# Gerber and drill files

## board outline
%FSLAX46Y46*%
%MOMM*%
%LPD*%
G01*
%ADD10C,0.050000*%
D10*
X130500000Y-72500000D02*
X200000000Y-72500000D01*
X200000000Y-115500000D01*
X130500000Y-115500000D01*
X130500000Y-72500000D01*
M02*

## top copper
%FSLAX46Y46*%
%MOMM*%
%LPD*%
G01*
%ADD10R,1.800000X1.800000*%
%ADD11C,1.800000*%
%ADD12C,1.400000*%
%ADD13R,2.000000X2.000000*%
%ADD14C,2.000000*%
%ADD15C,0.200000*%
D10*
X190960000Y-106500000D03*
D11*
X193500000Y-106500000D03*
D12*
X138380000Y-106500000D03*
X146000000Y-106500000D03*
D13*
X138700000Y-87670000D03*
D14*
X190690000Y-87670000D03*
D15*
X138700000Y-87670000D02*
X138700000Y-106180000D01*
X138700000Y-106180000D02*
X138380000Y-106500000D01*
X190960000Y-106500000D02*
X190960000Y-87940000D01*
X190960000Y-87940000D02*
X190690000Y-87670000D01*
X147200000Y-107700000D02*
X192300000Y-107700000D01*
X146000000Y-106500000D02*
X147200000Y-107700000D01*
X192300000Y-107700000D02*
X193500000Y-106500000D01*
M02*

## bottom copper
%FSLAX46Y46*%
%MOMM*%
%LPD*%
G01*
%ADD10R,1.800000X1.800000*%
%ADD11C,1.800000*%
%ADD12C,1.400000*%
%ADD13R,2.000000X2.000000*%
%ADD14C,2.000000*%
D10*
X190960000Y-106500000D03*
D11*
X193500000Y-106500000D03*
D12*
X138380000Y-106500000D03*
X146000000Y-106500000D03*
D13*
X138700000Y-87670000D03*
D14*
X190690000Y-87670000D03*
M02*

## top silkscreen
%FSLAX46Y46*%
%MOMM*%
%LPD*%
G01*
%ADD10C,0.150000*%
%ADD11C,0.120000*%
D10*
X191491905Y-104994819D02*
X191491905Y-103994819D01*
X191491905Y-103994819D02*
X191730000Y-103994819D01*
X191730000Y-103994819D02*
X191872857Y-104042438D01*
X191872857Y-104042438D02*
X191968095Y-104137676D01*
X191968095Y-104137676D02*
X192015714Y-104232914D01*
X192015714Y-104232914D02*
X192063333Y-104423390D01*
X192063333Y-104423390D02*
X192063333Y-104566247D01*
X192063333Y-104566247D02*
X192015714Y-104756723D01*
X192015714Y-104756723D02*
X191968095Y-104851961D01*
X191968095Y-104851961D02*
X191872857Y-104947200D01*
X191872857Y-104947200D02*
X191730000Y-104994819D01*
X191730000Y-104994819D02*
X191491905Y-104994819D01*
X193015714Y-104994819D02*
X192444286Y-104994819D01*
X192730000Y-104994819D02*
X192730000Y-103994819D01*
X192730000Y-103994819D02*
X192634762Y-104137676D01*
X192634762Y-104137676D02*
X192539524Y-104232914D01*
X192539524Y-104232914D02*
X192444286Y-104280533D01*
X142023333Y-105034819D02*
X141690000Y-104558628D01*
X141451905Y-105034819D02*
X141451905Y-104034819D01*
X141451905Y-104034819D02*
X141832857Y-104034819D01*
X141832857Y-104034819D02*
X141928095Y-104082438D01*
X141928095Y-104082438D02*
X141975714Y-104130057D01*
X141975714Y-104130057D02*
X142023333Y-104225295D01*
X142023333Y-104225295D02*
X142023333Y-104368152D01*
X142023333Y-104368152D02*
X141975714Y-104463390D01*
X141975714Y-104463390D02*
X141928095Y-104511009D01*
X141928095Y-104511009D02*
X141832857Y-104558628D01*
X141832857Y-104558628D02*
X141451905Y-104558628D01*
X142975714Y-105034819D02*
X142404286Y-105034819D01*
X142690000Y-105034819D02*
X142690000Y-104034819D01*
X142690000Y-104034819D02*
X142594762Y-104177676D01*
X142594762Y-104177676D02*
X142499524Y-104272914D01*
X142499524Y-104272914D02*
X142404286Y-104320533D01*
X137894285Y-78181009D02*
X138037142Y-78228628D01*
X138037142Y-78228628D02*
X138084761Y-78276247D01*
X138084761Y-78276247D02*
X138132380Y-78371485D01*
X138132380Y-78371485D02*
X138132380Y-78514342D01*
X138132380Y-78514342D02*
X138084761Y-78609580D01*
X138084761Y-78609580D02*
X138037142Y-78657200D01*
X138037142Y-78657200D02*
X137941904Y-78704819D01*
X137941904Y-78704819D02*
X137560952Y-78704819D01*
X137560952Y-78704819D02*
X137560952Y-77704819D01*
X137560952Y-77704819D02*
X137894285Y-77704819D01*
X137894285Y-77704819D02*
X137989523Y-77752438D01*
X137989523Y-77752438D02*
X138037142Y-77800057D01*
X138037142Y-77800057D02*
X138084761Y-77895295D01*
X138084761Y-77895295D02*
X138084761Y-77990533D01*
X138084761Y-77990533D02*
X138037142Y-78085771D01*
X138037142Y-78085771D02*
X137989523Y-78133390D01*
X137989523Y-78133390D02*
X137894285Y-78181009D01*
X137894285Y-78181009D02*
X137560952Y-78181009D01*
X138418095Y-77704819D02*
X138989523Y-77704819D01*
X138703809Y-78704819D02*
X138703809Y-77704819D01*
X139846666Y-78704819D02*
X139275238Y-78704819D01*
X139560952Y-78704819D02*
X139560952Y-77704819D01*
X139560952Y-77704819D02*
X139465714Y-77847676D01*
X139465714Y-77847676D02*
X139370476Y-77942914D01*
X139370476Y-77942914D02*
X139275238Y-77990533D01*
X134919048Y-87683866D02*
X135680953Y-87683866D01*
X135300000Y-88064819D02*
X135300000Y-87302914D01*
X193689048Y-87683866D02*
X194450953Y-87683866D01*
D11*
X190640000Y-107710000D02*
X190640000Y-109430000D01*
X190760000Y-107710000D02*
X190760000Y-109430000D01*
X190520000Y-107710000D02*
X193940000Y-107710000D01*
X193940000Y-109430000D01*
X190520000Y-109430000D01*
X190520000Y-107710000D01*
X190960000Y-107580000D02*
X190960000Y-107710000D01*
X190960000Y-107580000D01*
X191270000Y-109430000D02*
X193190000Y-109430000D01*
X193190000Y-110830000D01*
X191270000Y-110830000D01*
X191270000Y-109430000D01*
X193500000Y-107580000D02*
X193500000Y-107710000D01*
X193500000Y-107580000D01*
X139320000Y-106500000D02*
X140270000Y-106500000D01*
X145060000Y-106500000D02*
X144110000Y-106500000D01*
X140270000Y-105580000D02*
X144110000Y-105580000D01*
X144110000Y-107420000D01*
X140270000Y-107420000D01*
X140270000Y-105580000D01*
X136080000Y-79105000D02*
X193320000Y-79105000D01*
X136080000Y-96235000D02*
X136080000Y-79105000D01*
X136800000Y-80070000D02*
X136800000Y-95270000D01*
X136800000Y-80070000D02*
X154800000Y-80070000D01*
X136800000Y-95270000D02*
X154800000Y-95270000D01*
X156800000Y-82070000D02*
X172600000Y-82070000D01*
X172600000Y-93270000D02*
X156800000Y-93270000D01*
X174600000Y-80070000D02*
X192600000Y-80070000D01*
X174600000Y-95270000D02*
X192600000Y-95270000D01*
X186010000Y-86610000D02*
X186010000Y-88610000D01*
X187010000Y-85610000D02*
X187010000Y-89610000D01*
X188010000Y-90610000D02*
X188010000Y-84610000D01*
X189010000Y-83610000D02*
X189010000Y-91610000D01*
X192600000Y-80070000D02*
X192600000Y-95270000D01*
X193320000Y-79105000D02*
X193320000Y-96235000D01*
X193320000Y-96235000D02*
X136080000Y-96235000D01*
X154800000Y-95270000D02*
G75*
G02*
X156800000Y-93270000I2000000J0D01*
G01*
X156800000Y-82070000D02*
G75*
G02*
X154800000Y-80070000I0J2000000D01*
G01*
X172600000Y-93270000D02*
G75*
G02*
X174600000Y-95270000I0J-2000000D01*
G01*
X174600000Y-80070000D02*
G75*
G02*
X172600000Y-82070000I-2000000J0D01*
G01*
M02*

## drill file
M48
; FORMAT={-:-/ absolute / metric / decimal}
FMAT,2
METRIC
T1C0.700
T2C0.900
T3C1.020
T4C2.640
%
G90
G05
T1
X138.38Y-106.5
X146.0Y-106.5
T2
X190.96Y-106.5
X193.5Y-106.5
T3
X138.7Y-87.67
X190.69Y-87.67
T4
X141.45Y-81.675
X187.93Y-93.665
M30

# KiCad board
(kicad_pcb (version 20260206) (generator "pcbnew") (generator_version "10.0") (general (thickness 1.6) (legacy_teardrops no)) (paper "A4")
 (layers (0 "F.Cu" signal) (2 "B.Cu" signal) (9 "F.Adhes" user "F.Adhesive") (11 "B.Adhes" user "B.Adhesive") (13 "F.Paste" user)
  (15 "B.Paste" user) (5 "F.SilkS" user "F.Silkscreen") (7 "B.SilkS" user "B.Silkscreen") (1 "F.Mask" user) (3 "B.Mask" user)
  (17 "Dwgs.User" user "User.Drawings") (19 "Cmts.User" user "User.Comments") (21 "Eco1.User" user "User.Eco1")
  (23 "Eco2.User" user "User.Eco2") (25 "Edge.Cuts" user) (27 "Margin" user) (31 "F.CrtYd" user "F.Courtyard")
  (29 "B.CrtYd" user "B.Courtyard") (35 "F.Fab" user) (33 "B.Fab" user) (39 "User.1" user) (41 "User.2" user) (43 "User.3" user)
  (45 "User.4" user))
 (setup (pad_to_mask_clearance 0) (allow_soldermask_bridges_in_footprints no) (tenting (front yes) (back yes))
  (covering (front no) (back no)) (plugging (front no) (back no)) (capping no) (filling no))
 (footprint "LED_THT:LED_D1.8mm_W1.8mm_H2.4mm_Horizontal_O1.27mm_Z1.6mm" (layer "F.Cu") (at 190.96 106.5)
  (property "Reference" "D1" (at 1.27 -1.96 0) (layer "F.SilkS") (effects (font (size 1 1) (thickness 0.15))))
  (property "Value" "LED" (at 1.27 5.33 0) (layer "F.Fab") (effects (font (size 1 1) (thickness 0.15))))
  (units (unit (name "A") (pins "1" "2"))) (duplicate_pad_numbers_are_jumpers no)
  (fp_line (start -0.32 1.21) (end -0.32 2.93) (stroke (width 0.12) (type solid)) (layer "F.SilkS"))
  (fp_line (start -0.2 1.21) (end -0.2 2.93) (stroke (width 0.12) (type solid)) (layer "F.SilkS"))
  (fp_rect (start -0.44 1.21) (end 2.98 2.93) (stroke (width 0.12) (type solid)) (fill no) (layer "F.SilkS"))
  (fp_rect (start 0 1.08) (end 0 1.21) (stroke (width 0.12) (type solid)) (fill no) (layer "F.SilkS"))
  (fp_rect (start 0.31 2.93) (end 2.23 4.33) (stroke (width 0.12) (type solid)) (fill no) (layer "F.SilkS"))
  (fp_rect (start 2.54 1.08) (end 2.54 1.21) (stroke (width 0.12) (type solid)) (fill no) (layer "F.SilkS"))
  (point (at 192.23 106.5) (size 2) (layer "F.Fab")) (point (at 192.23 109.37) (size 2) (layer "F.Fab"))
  (pad "1" thru_hole rect (at 0 0) (size 1.8 1.8) (drill 0.9) (layers "*.Cu" "*.Mask") (remove_unused_layers no) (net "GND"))
  (pad "2" thru_hole circle (at 2.54 0) (size 1.8 1.8) (drill 0.9) (layers "*.Cu" "*.Mask") (remove_unused_layers no) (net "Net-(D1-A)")))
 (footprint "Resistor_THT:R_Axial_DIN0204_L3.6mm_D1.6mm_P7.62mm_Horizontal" (layer "F.Cu") (at 138.38 106.5)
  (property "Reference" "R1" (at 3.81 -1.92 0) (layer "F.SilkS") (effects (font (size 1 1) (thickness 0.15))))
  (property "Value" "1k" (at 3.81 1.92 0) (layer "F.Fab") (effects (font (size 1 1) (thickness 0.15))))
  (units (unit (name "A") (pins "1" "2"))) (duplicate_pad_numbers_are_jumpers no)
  (fp_line (start 0.94 0) (end 1.89 0) (stroke (width 0.12) (type solid)) (layer "F.SilkS"))
  (fp_line (start 6.68 0) (end 5.73 0) (stroke (width 0.12) (type solid)) (layer "F.SilkS"))
  (fp_rect (start 1.89 -0.92) (end 5.73 0.92) (stroke (width 0.12) (type solid)) (fill no) (layer "F.SilkS"))
  (pad "1" thru_hole circle (at 0 0) (size 1.4 1.4) (drill 0.7) (layers "*.Cu" "*.Mask") (remove_unused_layers no) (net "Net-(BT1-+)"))
  (pad "2" thru_hole circle (at 7.62 0) (size 1.4 1.4) (drill 0.7) (layers "*.Cu" "*.Mask") (remove_unused_layers no) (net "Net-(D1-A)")))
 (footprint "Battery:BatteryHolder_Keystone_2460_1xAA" (layer "F.Cu") (at 138.7 87.67)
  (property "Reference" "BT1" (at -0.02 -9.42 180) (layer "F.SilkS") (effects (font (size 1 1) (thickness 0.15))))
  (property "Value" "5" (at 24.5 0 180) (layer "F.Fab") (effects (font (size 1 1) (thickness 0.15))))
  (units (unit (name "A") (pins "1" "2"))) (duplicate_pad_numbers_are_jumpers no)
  (fp_line (start -2.62 -8.565) (end 54.62 -8.565) (stroke (width 0.12) (type solid)) (layer "F.SilkS"))
  (fp_line (start -2.62 8.565) (end -2.62 -8.565) (stroke (width 0.12) (type solid)) (layer "F.SilkS"))
  (fp_line (start -1.9 -7.6) (end -1.9 7.6) (stroke (width 0.12) (type solid)) (layer "F.SilkS"))
  (fp_line (start -1.9 -7.6) (end 16.1 -7.6) (stroke (width 0.12) (type solid)) (layer "F.SilkS"))
  (fp_line (start -1.9 7.6) (end 16.1 7.6) (stroke (width 0.12) (type solid)) (layer "F.SilkS"))
  (fp_line (start 18.1 -5.6) (end 33.9 -5.6) (stroke (width 0.12) (type solid)) (layer "F.SilkS"))
  (fp_line (start 33.9 5.6) (end 18.1 5.6) (stroke (width 0.12) (type solid)) (layer "F.SilkS"))
  (fp_line (start 35.9 -7.6) (end 53.9 -7.6) (stroke (width 0.12) (type solid)) (layer "F.SilkS"))
  (fp_line (start 35.9 7.6) (end 53.9 7.6) (stroke (width 0.12) (type solid)) (layer "F.SilkS"))
  (fp_line (start 47.31 -1.06) (end 47.31 0.94) (stroke (width 0.12) (type solid)) (layer "F.SilkS"))
  (fp_line (start 48.31 -2.06) (end 48.31 1.94) (stroke (width 0.12) (type solid)) (layer "F.SilkS"))
  (fp_line (start 49.31 2.94) (end 49.31 -3.06) (stroke (width 0.12) (type solid)) (layer "F.SilkS"))
  (fp_line (start 50.31 -4.06) (end 50.31 3.94) (stroke (width 0.12) (type solid)) (layer "F.SilkS"))
  (fp_line (start 53.9 -7.6) (end 53.9 7.6) (stroke (width 0.12) (type solid)) (layer "F.SilkS"))
  (fp_line (start 54.62 -8.565) (end 54.62 8.565) (stroke (width 0.12) (type solid)) (layer "F.SilkS"))
  (fp_line (start 54.62 8.565) (end -2.62 8.565) (stroke (width 0.12) (type solid)) (layer "F.SilkS"))
  (fp_arc (start 16.1 7.6) (mid 16.685786 6.185786) (end 18.1 5.6) (stroke (width 0.12) (type solid)) (layer "F.SilkS"))
  (fp_arc (start 18.1 -5.6) (mid 16.685786 -6.185786) (end 16.1 -7.6) (stroke (width 0.12) (type solid)) (layer "F.SilkS"))
  (fp_arc (start 33.9 5.6) (mid 35.314214 6.185786) (end 35.9 7.6) (stroke (width 0.12) (type solid)) (layer "F.SilkS"))
  (fp_arc (start 35.9 -7.6) (mid 35.314214 -6.185786) (end 33.9 -5.6) (stroke (width 0.12) (type solid)) (layer "F.SilkS"))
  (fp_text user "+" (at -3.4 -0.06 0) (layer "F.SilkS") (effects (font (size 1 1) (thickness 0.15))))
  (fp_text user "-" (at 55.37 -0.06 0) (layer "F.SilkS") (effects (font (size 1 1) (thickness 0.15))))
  (pad "" np_thru_hole circle (at 2.75 -5.995 90) (size 2.64 2.64) (drill 2.64) (layers "*.Cu" "*.Mask"))
  (pad "" np_thru_hole circle (at 49.23 5.995) (size 2.64 2.64) (drill 2.64) (layers "*.Cu" "*.Mask"))
  (pad "1" thru_hole rect (at 0 0 180) (size 2 2) (drill 1.02) (layers "*.Cu" "*.Mask") (remove_unused_layers no) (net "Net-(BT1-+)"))
  (pad "2" thru_hole circle (at 51.99 0 180) (size 2 2) (drill 1.02) (layers "*.Cu" "*.Mask") (remove_unused_layers no) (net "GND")))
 (gr_rect (start 130.5 72.5) (end 200 115.5) (stroke (width 0.05) (type default)) (fill no) (layer "Edge.Cuts"))
 (segment (start 138.7 87.67) (end 138.7 106.18) (width 0.2) (layer "F.Cu") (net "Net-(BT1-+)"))
 (segment (start 138.7 106.18) (end 138.38 106.5) (width 0.2) (layer "F.Cu") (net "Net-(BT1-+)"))
 (segment (start 190.96 106.5) (end 190.96 87.94) (width 0.2) (layer "F.Cu") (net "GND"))
 (segment (start 190.96 87.94) (end 190.69 87.67) (width 0.2) (layer "F.Cu") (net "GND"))
 (segment (start 147.2 107.7) (end 192.3 107.7) (width 0.2) (layer "F.Cu") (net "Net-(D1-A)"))
 (segment (start 146 106.5) (end 147.2 107.7) (width 0.2) (layer "F.Cu") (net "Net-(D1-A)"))
 (segment (start 192.3 107.7) (end 193.5 106.5) (width 0.2) (layer "F.Cu") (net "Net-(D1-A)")))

